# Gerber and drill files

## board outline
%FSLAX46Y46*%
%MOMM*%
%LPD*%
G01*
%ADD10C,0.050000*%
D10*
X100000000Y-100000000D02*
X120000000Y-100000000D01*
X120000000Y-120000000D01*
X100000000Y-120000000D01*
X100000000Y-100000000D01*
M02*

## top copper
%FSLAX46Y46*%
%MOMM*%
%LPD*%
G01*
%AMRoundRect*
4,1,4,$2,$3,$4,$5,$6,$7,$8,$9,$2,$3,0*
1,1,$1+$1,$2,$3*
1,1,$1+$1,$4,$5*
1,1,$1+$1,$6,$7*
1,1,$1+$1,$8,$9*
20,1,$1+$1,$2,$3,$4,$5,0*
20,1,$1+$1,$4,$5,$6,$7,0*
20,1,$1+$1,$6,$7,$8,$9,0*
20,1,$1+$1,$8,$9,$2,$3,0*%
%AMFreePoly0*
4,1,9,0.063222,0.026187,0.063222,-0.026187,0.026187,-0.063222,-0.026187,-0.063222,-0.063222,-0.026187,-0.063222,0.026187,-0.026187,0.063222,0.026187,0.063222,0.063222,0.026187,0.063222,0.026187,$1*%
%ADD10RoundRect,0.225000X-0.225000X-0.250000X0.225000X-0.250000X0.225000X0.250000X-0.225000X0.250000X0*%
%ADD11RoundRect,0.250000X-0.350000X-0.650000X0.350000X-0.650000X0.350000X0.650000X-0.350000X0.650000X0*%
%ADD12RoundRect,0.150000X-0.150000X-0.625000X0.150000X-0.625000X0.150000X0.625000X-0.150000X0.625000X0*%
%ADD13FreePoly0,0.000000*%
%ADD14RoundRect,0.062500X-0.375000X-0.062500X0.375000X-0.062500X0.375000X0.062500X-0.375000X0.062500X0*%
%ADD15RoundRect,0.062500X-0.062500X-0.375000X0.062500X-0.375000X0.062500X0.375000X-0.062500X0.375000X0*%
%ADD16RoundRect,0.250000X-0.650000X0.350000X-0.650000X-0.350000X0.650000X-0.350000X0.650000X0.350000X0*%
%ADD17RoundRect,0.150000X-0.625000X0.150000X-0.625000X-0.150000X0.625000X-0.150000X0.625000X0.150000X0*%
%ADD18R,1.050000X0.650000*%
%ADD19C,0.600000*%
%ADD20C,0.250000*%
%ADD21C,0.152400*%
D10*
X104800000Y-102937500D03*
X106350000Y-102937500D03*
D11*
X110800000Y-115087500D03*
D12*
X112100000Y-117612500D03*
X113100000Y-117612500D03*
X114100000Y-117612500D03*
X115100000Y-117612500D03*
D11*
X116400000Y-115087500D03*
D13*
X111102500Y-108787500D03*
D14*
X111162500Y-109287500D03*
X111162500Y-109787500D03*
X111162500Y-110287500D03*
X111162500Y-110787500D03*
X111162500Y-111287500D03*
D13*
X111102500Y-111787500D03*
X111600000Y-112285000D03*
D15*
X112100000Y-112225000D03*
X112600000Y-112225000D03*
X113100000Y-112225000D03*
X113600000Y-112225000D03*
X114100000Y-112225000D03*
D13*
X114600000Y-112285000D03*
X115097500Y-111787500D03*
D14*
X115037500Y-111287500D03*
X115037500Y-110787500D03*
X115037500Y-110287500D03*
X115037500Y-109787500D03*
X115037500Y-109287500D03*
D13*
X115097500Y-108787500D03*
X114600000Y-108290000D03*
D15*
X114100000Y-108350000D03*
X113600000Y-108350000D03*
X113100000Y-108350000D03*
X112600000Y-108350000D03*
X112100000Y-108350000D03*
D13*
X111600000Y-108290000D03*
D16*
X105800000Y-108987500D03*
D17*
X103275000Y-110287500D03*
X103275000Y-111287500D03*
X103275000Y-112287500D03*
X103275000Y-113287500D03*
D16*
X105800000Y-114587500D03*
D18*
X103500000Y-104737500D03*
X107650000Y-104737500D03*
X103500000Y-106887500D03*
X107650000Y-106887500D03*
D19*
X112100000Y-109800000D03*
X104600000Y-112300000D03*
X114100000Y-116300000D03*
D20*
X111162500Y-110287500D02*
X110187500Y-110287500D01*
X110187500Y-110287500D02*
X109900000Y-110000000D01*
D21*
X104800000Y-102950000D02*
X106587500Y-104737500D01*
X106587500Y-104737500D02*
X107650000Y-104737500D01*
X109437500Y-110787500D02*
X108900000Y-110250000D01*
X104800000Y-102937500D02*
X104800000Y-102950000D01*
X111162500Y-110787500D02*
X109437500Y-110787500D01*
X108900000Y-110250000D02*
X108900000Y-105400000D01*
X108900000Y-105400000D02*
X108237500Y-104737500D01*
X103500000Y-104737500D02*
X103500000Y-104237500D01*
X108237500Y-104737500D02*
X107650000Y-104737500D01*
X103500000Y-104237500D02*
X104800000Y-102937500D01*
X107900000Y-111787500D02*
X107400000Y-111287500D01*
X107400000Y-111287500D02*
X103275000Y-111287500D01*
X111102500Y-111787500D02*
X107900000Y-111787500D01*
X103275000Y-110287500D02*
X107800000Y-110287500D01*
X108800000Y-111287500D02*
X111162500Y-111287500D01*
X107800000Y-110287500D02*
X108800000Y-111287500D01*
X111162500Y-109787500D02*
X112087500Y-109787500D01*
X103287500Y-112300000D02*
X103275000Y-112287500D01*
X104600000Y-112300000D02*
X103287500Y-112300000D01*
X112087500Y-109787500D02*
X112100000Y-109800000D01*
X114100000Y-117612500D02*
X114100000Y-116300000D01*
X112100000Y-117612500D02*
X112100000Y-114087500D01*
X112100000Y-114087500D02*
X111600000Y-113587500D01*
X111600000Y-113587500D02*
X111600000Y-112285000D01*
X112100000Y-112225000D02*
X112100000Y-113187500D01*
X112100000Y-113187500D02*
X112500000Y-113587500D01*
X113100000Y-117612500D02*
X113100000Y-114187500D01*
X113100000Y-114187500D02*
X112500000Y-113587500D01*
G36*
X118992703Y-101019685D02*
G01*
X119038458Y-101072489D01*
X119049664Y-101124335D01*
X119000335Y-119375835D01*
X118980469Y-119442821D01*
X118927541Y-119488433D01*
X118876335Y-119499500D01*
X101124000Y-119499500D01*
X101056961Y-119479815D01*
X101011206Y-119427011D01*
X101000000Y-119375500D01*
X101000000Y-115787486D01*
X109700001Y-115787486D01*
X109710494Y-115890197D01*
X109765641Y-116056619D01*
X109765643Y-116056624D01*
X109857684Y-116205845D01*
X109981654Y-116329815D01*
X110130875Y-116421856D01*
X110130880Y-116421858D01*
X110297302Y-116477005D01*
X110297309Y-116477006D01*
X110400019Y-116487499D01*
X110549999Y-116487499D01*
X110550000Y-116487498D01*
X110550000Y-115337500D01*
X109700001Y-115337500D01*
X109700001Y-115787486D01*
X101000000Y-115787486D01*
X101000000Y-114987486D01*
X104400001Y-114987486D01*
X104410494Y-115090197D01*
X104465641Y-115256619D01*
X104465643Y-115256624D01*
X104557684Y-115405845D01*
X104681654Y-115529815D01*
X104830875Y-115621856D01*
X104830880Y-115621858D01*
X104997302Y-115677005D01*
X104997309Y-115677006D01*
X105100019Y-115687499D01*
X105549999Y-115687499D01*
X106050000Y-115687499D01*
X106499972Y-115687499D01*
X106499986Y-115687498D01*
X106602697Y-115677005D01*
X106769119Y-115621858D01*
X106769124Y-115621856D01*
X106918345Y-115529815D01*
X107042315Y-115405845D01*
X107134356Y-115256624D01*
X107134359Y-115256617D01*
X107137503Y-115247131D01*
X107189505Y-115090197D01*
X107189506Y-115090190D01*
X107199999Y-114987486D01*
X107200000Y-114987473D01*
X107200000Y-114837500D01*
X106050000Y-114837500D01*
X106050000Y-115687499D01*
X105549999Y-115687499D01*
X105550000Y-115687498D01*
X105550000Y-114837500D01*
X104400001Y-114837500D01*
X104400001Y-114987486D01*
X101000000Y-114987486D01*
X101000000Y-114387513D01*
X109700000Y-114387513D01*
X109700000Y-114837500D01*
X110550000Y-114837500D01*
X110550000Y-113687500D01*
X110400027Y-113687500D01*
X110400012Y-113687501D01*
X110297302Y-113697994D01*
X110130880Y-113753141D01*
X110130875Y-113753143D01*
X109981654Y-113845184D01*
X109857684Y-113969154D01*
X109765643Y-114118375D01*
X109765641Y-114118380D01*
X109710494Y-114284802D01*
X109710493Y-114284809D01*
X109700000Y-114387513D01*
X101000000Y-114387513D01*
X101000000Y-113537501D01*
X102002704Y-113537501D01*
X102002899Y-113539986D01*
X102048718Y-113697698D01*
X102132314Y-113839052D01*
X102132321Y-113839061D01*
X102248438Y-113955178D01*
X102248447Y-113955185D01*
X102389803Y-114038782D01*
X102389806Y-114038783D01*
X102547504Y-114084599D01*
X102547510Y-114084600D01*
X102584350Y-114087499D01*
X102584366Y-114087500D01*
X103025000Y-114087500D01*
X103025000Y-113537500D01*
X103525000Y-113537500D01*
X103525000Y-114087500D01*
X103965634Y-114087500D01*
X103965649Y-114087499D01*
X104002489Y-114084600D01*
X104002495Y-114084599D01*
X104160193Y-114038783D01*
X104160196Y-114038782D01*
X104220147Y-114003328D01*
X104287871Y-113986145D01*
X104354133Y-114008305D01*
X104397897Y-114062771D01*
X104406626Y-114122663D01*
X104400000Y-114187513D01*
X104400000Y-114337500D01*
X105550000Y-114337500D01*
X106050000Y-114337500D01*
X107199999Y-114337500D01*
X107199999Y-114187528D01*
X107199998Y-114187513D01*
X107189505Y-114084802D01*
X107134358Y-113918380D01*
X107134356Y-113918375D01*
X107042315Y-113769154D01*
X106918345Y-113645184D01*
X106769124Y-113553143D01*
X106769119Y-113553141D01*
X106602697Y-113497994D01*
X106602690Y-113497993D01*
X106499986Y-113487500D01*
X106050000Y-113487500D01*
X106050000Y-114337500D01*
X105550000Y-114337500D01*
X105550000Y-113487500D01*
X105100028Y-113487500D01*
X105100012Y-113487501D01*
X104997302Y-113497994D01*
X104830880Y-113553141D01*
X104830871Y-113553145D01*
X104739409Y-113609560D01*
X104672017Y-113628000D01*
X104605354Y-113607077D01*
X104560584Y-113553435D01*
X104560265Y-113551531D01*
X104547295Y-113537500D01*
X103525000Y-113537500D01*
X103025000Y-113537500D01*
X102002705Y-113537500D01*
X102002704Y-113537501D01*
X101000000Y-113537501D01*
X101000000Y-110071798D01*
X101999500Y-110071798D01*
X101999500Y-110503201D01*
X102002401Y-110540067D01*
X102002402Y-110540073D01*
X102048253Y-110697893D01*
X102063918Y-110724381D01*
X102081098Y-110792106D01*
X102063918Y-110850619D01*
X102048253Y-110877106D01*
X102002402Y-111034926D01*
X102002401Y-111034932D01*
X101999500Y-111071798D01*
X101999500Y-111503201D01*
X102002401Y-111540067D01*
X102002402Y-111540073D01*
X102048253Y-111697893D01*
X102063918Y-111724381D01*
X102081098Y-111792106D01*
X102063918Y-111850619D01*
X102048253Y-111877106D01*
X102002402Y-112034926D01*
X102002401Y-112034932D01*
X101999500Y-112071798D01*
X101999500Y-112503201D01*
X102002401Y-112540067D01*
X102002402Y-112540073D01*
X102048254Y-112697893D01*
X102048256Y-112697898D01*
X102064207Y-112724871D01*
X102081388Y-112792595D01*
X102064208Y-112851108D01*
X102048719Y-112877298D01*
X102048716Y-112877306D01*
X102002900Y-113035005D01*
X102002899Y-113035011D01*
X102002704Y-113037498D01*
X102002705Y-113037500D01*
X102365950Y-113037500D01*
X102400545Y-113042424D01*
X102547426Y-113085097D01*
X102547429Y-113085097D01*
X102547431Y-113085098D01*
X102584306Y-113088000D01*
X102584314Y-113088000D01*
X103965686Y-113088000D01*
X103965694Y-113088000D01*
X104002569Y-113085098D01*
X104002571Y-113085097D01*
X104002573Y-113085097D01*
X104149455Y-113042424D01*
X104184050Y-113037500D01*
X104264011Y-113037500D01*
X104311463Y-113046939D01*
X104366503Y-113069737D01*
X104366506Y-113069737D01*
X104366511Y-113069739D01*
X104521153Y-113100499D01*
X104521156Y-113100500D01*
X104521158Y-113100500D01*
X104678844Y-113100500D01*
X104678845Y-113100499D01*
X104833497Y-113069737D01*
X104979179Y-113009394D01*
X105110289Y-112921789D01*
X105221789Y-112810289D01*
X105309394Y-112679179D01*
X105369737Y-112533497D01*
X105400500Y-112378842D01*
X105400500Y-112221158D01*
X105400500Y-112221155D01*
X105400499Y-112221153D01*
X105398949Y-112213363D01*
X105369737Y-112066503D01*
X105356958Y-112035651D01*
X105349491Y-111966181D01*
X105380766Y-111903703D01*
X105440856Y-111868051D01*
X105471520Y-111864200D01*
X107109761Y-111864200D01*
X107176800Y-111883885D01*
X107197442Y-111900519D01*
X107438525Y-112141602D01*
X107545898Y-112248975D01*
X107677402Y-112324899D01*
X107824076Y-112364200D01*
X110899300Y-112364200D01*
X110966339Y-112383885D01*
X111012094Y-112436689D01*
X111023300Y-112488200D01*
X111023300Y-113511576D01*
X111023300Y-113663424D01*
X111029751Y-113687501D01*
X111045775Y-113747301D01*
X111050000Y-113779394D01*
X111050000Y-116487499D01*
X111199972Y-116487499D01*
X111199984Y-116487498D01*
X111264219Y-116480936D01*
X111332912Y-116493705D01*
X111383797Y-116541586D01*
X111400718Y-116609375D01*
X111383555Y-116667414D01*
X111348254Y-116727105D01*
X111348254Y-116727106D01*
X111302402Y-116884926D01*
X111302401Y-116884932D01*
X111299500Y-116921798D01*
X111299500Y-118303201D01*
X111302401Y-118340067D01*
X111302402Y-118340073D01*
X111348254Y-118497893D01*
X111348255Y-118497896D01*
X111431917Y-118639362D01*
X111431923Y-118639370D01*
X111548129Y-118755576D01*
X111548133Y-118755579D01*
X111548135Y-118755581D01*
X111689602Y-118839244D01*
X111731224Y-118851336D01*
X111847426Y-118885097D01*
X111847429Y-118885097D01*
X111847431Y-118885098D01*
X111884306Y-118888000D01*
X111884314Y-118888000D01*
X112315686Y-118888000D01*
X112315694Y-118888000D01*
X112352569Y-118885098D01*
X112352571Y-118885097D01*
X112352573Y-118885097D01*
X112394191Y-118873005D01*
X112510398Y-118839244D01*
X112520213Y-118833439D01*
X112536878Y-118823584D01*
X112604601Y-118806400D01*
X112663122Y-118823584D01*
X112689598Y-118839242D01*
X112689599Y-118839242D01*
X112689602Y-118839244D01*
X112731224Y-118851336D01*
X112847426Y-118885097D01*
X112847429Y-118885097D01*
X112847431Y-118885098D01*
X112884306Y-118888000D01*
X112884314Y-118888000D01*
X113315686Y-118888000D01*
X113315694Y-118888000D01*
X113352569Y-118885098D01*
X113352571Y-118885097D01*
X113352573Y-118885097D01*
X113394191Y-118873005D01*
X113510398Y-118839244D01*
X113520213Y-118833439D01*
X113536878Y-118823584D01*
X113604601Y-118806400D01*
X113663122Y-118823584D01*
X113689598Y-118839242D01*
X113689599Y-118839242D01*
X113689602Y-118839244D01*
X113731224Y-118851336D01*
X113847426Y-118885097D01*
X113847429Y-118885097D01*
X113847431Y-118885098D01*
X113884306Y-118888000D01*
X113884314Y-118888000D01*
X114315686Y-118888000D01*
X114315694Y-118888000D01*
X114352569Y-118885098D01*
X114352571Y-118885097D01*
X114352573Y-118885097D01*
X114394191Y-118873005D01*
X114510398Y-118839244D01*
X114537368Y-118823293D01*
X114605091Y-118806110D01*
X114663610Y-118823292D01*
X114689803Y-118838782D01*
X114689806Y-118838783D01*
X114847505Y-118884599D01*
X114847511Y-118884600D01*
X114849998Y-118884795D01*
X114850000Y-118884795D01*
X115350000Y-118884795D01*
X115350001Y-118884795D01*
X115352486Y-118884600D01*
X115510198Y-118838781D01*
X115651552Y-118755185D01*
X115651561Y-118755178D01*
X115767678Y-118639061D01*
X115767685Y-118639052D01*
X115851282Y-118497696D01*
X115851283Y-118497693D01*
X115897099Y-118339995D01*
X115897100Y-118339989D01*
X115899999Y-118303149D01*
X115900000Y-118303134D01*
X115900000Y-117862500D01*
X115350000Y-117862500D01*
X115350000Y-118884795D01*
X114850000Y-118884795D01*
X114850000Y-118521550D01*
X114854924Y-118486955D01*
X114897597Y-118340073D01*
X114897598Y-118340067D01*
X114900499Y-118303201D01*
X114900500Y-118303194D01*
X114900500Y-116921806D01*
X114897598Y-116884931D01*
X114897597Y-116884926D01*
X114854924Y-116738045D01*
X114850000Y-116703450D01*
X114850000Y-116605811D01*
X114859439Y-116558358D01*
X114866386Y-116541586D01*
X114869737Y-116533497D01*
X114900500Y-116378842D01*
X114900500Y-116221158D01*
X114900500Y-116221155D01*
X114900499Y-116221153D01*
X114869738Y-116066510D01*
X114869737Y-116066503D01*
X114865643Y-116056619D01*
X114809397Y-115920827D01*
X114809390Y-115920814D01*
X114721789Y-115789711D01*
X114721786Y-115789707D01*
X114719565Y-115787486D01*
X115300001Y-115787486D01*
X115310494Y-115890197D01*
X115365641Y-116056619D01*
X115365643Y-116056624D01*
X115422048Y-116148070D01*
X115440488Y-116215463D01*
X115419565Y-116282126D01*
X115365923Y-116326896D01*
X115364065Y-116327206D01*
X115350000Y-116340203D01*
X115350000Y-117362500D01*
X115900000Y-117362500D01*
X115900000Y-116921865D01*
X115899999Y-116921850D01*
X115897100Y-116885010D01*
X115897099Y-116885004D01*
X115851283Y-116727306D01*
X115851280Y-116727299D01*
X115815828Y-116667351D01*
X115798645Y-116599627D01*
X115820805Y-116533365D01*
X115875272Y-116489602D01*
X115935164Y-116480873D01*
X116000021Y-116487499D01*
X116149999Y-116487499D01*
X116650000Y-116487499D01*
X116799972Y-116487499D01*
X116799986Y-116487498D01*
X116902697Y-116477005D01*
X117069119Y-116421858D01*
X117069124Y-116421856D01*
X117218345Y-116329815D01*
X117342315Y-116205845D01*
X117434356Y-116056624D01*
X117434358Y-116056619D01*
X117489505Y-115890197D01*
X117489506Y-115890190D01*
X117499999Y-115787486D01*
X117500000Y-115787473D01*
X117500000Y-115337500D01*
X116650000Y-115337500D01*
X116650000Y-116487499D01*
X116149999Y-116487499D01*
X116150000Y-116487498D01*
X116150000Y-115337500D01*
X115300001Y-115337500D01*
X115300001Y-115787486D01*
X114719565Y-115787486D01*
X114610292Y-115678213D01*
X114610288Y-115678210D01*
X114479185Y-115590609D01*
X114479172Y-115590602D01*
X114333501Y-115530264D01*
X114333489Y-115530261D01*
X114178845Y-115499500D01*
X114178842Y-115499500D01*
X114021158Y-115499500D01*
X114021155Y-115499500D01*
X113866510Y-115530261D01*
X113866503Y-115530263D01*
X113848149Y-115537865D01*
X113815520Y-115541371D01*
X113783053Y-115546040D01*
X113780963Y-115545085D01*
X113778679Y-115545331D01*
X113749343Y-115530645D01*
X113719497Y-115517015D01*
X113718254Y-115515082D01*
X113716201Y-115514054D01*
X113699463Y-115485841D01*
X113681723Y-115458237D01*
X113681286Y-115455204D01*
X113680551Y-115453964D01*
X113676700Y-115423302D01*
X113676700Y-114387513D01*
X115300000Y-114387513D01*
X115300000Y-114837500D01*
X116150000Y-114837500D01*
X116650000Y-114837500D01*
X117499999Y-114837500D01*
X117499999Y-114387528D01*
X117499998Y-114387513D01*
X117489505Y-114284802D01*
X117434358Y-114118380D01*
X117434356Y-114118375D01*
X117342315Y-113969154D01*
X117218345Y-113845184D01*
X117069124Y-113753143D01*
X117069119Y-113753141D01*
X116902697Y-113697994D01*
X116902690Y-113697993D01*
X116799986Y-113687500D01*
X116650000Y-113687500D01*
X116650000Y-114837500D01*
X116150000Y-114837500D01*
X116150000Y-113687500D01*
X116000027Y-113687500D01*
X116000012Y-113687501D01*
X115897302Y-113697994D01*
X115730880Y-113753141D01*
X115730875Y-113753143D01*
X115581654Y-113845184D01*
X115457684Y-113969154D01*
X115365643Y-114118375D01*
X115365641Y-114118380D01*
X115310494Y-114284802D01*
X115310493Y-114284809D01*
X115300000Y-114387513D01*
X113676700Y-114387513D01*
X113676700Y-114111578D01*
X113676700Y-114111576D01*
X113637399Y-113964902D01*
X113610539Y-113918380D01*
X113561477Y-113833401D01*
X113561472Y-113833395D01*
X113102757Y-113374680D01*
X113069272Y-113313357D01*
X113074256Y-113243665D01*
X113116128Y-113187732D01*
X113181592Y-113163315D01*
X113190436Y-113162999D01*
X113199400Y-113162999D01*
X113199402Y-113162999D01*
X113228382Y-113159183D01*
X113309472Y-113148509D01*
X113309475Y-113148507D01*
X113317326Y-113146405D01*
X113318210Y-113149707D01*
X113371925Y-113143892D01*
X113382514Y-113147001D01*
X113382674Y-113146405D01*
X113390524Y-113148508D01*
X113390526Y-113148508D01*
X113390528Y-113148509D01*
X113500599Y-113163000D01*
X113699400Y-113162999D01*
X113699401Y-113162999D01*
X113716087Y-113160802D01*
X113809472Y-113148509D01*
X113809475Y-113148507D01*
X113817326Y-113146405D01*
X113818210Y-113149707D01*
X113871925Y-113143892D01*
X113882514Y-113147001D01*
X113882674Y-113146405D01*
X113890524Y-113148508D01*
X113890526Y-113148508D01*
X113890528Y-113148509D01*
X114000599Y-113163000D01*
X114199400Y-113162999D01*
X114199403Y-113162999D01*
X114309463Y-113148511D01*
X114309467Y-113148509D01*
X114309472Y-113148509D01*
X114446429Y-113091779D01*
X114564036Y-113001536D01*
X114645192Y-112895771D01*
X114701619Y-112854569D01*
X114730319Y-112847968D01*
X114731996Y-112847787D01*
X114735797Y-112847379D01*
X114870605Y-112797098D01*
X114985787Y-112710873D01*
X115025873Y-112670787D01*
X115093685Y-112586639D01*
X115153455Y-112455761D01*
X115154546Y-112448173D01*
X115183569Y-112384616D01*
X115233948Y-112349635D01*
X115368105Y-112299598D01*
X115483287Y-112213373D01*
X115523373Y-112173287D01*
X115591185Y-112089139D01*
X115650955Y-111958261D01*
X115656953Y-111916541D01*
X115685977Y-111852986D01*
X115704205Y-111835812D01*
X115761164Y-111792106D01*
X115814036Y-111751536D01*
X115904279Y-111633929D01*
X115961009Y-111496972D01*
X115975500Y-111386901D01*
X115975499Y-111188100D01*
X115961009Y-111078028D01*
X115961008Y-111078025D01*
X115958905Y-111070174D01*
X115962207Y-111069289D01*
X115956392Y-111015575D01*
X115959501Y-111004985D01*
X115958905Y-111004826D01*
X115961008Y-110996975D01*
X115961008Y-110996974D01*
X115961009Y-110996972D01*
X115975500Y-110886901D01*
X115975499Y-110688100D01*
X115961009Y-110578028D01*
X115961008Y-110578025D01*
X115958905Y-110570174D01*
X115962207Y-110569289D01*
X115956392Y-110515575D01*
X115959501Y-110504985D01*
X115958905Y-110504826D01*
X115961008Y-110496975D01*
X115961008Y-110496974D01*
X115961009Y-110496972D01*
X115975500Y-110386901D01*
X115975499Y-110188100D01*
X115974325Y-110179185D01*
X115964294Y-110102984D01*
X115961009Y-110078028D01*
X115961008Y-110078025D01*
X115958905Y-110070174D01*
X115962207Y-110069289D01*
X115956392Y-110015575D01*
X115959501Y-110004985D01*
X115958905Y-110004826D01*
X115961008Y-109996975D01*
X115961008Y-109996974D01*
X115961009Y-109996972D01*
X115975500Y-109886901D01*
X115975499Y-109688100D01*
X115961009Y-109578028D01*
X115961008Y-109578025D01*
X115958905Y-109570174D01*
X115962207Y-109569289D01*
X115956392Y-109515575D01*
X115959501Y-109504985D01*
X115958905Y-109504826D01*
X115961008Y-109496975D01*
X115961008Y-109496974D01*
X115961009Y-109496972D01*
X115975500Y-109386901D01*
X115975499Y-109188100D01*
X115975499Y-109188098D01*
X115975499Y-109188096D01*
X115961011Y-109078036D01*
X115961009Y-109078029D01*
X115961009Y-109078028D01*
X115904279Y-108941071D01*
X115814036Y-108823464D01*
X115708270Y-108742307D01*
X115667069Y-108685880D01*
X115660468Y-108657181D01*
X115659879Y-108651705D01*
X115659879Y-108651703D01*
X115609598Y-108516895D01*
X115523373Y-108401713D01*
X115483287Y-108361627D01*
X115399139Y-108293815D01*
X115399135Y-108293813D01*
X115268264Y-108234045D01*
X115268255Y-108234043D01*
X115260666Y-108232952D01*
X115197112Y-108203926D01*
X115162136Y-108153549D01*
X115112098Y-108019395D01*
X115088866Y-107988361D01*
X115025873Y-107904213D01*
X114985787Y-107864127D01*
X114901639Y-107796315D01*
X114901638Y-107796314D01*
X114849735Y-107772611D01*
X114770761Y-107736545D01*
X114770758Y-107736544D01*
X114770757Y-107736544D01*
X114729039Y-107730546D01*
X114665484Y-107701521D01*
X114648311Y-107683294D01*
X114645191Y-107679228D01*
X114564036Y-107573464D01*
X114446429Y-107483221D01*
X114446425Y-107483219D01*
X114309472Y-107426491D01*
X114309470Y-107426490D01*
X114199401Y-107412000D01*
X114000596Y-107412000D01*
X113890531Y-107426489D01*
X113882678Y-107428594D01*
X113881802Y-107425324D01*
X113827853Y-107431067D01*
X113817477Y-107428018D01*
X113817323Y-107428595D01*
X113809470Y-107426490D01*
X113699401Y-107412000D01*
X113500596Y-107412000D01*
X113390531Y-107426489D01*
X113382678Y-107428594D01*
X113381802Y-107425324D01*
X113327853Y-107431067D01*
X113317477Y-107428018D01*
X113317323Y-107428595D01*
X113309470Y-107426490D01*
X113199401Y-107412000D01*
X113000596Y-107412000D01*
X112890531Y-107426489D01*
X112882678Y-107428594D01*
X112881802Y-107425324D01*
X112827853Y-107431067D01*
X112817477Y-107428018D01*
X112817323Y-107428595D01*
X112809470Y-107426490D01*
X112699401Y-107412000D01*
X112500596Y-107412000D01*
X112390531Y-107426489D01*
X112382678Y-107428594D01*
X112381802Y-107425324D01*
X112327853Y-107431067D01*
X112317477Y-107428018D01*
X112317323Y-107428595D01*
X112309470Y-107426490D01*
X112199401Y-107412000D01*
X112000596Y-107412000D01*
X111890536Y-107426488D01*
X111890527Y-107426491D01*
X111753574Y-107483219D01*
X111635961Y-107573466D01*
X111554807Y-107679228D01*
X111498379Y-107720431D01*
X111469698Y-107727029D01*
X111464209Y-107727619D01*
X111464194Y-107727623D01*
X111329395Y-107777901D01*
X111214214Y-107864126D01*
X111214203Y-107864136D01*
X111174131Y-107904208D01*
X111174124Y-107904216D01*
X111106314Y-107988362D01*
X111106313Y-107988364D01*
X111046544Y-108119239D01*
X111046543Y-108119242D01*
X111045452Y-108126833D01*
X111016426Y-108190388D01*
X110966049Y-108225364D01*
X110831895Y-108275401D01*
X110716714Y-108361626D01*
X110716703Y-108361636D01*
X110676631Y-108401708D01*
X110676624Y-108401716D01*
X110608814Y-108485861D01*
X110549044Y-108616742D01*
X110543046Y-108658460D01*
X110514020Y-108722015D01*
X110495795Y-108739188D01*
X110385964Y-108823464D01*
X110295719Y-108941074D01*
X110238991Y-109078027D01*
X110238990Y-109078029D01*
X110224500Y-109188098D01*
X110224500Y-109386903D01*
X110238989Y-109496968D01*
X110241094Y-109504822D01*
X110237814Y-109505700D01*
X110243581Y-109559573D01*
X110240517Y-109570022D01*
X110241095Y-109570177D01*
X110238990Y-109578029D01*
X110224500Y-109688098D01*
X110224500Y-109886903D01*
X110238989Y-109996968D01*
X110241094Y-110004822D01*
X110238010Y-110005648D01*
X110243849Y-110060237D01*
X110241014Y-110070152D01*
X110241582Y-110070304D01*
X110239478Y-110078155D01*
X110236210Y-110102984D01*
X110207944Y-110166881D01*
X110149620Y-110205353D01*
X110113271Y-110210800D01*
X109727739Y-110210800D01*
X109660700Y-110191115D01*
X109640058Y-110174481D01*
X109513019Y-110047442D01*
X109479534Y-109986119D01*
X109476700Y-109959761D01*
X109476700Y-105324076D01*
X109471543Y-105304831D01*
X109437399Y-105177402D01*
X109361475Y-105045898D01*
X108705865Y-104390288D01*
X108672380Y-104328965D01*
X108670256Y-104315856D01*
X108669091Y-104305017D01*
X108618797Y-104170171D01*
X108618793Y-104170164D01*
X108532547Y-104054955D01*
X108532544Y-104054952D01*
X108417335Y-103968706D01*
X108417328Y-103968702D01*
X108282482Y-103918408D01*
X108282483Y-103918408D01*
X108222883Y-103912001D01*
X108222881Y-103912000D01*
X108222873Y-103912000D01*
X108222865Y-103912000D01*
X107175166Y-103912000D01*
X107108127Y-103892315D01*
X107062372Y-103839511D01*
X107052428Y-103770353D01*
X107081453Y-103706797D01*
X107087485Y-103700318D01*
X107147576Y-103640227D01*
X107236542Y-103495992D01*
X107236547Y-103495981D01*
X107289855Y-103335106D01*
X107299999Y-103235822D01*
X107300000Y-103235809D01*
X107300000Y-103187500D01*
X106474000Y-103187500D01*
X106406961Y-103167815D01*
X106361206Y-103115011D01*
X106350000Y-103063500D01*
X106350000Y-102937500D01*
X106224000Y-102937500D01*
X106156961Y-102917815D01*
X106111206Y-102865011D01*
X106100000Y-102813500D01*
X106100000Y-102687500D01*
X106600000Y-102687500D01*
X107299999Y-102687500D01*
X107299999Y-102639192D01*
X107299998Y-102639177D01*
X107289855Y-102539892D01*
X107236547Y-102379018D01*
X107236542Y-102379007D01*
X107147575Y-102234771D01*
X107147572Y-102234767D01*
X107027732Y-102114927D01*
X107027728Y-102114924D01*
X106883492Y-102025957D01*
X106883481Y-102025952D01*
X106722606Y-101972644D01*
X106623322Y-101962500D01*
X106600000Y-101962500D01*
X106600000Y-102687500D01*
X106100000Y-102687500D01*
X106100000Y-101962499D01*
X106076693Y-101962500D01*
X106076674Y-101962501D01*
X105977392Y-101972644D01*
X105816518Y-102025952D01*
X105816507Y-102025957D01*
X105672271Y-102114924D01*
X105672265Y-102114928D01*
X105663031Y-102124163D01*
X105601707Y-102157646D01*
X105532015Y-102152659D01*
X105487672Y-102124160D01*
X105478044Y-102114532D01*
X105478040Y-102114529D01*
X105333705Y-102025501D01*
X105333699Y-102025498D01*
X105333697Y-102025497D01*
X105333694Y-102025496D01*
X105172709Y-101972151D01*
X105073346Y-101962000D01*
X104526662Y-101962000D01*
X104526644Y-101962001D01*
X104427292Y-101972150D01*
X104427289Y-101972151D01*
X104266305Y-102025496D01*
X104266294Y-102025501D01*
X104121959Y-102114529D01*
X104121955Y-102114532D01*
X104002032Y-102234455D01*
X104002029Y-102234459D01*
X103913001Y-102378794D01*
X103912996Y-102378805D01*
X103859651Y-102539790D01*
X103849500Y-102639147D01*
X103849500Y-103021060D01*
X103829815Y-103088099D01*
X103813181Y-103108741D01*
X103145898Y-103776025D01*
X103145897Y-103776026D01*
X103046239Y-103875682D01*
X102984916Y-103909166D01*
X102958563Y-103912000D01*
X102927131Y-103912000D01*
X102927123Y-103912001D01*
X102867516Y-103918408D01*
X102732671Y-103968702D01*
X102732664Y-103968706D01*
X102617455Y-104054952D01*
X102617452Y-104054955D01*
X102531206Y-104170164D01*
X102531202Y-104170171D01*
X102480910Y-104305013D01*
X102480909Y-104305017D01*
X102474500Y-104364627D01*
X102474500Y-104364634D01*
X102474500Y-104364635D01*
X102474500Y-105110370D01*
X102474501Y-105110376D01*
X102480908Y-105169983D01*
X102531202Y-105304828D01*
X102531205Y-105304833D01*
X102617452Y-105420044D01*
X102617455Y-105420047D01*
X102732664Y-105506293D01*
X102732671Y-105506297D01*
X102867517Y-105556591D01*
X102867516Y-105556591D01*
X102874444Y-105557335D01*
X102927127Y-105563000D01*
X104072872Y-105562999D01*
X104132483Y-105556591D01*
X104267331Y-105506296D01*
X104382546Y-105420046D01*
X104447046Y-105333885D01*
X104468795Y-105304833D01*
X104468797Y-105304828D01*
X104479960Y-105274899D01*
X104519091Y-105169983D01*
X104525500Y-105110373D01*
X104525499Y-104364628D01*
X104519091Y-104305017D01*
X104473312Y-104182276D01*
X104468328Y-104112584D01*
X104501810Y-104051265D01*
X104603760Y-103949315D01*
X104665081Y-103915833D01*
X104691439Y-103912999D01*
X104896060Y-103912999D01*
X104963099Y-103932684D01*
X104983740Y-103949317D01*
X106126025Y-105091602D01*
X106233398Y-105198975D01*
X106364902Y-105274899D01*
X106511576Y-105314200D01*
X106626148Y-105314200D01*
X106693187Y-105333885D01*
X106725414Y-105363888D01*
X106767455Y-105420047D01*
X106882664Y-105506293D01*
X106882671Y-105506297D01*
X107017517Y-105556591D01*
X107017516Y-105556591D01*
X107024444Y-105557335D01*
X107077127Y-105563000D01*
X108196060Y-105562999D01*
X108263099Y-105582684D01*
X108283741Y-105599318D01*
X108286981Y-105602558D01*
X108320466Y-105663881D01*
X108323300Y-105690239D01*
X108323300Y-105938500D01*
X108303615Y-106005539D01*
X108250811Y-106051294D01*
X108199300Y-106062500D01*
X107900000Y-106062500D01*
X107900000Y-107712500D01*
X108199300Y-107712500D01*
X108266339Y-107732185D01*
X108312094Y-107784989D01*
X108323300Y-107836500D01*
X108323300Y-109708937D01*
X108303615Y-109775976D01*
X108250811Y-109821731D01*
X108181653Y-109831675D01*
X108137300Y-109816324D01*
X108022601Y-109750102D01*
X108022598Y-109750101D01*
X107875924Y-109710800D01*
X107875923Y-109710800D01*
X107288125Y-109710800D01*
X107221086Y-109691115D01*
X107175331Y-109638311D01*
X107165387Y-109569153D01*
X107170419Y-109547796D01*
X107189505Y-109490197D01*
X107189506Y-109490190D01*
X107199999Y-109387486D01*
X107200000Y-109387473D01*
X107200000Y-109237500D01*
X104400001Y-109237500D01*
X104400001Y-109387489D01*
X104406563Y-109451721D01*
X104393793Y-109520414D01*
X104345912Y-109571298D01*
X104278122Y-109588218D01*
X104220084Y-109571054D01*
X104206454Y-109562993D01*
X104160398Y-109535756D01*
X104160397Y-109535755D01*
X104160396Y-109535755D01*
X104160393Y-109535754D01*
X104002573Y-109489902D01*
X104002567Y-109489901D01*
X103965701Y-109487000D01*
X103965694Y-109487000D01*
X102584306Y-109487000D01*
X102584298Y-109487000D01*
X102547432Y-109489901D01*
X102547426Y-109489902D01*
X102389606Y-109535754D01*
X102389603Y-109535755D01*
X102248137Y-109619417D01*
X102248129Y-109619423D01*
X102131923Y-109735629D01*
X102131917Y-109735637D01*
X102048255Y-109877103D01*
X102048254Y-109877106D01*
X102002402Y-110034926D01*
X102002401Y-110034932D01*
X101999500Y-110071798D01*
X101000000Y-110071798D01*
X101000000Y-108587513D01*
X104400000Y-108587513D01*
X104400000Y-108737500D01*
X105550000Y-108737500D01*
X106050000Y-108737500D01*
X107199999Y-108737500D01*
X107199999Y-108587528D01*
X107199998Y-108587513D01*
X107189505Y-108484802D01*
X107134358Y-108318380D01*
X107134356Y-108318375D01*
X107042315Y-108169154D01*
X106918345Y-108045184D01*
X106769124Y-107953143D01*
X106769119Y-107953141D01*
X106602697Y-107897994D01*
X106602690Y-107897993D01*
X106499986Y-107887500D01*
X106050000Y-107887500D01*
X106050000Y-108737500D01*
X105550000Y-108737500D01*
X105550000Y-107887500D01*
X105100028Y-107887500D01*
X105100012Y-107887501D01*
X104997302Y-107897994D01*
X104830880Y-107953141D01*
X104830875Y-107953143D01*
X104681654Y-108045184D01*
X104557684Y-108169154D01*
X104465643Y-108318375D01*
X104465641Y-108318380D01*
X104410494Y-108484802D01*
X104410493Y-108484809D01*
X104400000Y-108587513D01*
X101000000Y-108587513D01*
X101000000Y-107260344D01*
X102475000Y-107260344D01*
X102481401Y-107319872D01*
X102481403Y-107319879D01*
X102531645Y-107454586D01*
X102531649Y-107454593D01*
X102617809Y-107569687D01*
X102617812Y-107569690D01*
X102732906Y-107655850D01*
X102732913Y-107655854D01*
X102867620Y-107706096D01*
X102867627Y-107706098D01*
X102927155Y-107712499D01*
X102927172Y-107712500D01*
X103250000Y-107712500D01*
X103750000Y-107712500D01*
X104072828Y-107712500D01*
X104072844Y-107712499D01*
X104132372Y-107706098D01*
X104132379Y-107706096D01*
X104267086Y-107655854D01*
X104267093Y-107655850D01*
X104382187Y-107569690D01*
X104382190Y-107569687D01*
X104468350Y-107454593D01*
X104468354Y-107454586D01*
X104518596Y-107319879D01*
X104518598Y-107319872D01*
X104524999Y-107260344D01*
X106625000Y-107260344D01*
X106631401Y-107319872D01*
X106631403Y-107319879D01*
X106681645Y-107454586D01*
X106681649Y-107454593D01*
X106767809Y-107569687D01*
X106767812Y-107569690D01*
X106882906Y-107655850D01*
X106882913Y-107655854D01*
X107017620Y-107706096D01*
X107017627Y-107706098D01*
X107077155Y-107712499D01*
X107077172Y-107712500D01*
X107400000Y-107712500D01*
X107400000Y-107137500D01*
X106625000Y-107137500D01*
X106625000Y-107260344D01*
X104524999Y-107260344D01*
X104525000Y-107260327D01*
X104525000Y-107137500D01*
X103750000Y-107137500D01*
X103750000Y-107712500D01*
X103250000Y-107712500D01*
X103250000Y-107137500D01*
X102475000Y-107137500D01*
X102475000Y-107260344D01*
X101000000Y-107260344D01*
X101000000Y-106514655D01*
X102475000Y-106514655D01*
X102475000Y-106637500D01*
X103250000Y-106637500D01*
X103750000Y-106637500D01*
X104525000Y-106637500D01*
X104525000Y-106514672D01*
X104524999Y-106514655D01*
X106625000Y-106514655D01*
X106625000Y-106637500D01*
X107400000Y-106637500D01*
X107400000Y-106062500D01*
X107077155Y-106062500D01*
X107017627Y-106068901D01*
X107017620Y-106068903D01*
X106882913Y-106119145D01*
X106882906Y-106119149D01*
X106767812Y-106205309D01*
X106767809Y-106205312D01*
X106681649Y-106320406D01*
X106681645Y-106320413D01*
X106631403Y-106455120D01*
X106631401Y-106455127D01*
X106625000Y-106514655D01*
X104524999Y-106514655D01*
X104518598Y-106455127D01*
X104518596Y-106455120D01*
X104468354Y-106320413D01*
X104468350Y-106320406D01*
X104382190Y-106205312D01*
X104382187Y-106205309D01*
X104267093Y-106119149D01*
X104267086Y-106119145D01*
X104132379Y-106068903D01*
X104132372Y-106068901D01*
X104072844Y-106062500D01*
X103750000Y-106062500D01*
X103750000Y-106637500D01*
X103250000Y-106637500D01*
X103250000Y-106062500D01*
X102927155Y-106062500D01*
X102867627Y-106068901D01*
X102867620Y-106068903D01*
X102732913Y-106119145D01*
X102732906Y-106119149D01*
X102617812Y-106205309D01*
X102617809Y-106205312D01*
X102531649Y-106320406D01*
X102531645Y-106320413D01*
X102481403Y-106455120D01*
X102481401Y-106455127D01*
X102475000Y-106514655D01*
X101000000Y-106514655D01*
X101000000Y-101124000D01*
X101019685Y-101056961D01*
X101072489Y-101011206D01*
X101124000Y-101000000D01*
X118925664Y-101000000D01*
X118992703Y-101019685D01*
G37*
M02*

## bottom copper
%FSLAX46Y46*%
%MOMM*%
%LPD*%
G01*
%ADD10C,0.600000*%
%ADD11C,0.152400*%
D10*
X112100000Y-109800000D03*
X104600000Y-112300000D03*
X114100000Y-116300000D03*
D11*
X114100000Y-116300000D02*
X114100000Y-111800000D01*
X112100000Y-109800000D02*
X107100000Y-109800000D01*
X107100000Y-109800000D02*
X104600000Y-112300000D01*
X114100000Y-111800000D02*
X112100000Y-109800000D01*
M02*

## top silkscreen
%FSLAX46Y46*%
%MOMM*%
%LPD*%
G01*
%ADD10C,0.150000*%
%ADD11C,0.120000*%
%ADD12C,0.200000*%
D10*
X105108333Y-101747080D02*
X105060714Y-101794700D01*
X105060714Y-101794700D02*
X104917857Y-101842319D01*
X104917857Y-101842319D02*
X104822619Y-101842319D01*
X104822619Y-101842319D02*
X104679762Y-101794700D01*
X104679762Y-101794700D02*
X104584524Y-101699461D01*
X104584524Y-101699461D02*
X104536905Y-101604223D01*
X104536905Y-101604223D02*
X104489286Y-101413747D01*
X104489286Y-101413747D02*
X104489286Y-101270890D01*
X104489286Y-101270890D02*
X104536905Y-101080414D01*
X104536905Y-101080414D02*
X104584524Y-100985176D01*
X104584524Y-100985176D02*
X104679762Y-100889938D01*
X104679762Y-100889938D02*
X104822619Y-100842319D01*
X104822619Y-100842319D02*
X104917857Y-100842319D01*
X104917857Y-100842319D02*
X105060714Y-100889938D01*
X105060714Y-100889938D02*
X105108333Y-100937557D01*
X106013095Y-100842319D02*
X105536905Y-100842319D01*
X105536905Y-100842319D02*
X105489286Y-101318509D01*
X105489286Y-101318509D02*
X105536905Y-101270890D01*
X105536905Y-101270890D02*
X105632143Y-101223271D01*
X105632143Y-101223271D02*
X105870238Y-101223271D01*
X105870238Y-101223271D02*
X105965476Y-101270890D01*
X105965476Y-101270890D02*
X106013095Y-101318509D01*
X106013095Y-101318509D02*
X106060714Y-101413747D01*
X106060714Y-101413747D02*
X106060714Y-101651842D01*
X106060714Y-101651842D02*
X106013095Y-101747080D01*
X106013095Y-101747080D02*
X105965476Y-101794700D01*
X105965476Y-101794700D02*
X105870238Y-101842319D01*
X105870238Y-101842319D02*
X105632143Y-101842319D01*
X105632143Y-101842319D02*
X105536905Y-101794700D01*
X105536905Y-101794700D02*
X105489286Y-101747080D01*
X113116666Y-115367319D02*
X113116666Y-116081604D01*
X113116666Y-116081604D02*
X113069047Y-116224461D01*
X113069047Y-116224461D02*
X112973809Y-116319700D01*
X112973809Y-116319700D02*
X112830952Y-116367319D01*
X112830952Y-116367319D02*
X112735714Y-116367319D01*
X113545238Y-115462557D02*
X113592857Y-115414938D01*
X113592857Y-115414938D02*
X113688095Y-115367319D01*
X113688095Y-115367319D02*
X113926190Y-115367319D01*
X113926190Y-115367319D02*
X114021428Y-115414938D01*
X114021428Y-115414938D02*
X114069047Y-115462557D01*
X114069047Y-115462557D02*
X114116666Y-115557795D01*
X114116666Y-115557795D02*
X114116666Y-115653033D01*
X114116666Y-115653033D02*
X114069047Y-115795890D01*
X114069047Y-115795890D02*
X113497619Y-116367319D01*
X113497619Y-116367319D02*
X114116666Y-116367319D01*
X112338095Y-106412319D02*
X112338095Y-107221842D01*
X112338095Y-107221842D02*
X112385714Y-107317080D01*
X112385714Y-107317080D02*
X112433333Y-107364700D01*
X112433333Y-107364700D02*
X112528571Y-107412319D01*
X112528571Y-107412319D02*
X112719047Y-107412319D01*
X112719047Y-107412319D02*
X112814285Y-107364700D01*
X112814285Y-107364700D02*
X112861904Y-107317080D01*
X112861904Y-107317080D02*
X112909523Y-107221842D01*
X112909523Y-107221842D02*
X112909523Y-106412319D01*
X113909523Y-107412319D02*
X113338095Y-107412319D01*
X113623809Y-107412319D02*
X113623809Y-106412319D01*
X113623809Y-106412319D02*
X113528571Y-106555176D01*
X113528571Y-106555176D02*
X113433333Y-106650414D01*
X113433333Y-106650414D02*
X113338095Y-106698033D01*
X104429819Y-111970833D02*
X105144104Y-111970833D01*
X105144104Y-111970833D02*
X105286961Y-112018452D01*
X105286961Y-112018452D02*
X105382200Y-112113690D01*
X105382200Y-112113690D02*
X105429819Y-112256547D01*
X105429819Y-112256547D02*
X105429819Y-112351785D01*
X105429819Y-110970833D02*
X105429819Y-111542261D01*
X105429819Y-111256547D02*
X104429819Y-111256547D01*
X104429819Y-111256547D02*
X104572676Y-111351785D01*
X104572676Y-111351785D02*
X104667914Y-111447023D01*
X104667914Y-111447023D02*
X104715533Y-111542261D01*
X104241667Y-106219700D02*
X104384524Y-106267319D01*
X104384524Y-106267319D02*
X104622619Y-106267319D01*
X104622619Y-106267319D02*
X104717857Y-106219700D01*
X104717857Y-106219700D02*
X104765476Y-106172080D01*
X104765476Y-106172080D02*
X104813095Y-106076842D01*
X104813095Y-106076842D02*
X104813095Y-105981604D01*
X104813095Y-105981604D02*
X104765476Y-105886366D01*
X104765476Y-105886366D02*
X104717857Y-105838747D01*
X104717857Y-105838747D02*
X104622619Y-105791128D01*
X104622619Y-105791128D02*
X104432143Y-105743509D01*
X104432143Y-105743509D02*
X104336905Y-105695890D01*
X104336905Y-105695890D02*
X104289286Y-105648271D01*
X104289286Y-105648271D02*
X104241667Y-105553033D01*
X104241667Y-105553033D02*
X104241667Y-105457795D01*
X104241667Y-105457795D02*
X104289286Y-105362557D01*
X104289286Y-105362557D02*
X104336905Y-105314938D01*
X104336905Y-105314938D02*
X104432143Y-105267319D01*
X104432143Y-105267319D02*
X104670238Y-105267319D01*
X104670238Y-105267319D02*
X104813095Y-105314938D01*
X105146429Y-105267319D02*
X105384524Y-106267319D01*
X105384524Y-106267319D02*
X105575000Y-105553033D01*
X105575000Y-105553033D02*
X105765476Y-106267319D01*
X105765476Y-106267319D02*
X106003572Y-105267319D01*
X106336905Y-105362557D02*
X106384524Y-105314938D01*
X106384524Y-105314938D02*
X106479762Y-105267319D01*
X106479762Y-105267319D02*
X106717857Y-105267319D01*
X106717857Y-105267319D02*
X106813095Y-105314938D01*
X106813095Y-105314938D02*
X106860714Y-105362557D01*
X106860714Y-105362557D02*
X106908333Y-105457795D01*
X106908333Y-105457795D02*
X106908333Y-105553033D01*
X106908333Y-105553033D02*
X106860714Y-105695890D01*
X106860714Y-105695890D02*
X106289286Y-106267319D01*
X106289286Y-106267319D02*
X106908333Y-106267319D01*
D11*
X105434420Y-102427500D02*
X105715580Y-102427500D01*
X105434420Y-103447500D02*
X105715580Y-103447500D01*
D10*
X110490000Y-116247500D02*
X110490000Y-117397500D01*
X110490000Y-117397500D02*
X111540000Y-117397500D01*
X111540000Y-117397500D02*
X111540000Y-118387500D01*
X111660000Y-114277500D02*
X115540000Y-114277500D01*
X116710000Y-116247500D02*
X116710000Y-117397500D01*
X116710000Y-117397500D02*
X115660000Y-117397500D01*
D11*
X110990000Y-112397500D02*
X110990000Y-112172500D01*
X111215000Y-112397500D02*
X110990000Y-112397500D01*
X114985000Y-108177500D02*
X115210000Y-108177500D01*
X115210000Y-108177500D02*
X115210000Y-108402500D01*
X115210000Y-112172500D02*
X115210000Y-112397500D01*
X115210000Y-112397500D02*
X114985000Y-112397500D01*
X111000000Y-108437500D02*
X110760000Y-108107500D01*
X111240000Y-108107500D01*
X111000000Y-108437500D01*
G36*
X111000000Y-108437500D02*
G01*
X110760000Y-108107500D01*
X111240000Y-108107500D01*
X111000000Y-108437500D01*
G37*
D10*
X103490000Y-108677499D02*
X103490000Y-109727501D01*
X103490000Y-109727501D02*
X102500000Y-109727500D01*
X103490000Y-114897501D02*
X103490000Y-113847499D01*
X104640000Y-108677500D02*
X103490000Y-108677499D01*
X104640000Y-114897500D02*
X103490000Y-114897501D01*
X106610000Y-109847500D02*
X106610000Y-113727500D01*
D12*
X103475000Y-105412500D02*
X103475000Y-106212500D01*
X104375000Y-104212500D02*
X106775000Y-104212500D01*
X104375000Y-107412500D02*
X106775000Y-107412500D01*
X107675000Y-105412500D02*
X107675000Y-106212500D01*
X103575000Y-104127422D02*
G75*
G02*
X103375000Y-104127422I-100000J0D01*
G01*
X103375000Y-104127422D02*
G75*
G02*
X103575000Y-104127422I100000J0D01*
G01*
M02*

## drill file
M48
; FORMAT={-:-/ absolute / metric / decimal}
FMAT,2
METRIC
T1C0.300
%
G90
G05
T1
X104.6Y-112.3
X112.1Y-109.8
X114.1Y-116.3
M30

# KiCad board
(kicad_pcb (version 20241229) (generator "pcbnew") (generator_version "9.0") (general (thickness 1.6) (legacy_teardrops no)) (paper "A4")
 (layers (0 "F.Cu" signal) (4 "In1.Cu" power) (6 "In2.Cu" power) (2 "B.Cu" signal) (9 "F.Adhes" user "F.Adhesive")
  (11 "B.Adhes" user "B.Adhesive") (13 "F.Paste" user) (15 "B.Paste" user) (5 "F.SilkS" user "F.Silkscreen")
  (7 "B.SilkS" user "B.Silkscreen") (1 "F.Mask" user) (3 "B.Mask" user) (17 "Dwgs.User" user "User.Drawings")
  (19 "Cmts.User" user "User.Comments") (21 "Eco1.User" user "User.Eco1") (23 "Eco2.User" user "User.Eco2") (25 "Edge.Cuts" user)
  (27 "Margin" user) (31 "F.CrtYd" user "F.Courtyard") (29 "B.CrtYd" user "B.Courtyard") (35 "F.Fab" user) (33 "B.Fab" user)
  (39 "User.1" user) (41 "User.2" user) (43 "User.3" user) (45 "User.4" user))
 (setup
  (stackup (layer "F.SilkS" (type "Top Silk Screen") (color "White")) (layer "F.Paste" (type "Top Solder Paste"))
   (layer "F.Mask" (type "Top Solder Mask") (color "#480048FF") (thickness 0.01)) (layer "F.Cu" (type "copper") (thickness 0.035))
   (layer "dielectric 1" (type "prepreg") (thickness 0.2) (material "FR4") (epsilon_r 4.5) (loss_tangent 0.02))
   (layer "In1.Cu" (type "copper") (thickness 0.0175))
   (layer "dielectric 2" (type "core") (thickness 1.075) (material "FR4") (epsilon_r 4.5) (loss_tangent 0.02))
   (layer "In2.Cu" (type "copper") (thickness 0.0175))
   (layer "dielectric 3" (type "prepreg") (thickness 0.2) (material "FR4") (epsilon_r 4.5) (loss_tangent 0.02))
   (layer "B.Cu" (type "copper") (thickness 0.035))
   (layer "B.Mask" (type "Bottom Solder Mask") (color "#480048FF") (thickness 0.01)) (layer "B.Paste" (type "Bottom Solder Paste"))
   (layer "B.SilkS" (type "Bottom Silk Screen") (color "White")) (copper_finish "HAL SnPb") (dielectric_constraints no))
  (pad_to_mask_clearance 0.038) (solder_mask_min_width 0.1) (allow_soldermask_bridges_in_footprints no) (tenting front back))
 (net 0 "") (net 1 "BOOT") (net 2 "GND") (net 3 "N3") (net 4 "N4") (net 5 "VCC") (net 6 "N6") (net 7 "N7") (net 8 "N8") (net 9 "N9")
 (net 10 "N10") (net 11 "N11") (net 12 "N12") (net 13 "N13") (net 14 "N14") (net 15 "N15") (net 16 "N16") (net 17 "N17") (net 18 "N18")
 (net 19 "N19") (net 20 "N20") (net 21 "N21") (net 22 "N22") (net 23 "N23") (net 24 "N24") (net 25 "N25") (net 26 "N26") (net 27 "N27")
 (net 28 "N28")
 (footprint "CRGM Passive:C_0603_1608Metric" (layer "F.Cu") (at 105.575 102.9375)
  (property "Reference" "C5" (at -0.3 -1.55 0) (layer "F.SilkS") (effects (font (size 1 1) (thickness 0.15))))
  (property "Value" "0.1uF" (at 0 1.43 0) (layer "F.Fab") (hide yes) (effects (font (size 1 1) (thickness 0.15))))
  (fp_line (start -0.14058 -0.51) (end 0.14058 -0.51) (stroke (width 0.12) (type solid)) (layer "F.SilkS"))
  (fp_line (start -0.14058 0.51) (end 0.14058 0.51) (stroke (width 0.12) (type solid)) (layer "F.SilkS"))
  (pad "1" smd roundrect (at -0.775 0) (size 0.9 0.95) (layers "F.Cu" "F.Mask" "F.Paste") (roundrect_rratio 0.25) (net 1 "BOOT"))
  (pad "2" smd roundrect (at 0.775 0) (size 0.9 0.95) (layers "F.Cu" "F.Mask" "F.Paste") (roundrect_rratio 0.25) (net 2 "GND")))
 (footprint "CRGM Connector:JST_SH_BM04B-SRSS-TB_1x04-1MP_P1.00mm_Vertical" (layer "F.Cu") (at 113.6 116.2875)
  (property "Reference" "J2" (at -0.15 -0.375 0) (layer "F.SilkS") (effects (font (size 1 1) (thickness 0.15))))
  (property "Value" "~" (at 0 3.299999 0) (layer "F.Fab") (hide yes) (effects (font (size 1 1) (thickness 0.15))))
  (fp_line (start -3.11 -0.04) (end -3.11 1.11) (stroke (width 0.15) (type solid)) (layer "F.SilkS"))
  (fp_line (start -3.11 1.11) (end -2.06 1.11) (stroke (width 0.15) (type solid)) (layer "F.SilkS"))
  (fp_line (start -2.06 1.11) (end -2.06 2.1) (stroke (width 0.15) (type solid)) (layer "F.SilkS"))
  (fp_line (start -1.94 -2.01) (end 1.94 -2.01) (stroke (width 0.15) (type solid)) (layer "F.SilkS"))
  (fp_line (start 3.11 -0.04) (end 3.11 1.11) (stroke (width 0.15) (type solid)) (layer "F.SilkS"))
  (fp_line (start 3.11 1.11) (end 2.06 1.11) (stroke (width 0.15) (type solid)) (layer "F.SilkS"))
  (pad "0" smd roundrect (at -2.8 -1.2) (size 1.2 1.8) (layers "F.Cu" "F.Mask" "F.Paste") (roundrect_rratio 0.208333) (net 2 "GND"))
  (pad "1" smd roundrect (at -1.5 1.325) (size 0.6 1.55) (layers "F.Cu" "F.Mask" "F.Paste") (roundrect_rratio 0.25) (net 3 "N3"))
  (pad "2" smd roundrect (at -0.5 1.325) (size 0.6 1.55) (layers "F.Cu" "F.Mask" "F.Paste") (roundrect_rratio 0.25) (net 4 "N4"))
  (pad "3" smd roundrect (at 0.5 1.325) (size 0.6 1.55) (layers "F.Cu" "F.Mask" "F.Paste") (roundrect_rratio 0.25) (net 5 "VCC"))
  (pad "4" smd roundrect (at 1.5 1.325) (size 0.6 1.55) (layers "F.Cu" "F.Mask" "F.Paste") (roundrect_rratio 0.25) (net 2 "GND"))
  (pad "5" smd roundrect (at 2.8 -1.2) (size 1.2 1.8) (layers "F.Cu" "F.Mask" "F.Paste") (roundrect_rratio 0.208333) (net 2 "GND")))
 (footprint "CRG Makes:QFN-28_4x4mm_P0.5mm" (layer "F.Cu") (at 113.1 110.2875)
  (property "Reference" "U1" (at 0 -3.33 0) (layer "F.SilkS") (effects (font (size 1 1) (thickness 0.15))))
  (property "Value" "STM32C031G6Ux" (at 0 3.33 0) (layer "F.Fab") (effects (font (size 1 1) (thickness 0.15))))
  (fp_line (start -2.11 2.11) (end -2.11 1.885) (stroke (width 0.12) (type solid)) (layer "F.SilkS"))
  (fp_line (start -1.885 2.11) (end -2.11 2.11) (stroke (width 0.12) (type solid)) (layer "F.SilkS"))
  (fp_line (start 1.885 -2.11) (end 2.11 -2.11) (stroke (width 0.12) (type solid)) (layer "F.SilkS"))
  (fp_line (start 2.11 -2.11) (end 2.11 -1.885) (stroke (width 0.12) (type solid)) (layer "F.SilkS"))
  (fp_line (start 2.11 1.885) (end 2.11 2.11) (stroke (width 0.12) (type solid)) (layer "F.SilkS"))
  (fp_line (start 2.11 2.11) (end 1.885 2.11) (stroke (width 0.12) (type solid)) (layer "F.SilkS"))
  (fp_poly (pts (xy -2.1 -1.85) (xy -2.34 -2.18) (xy -1.86 -2.18)) (stroke (width 0.12) (type solid)) (fill yes) (layer "F.SilkS"))
  (pad "1" smd custom (at -1.9975 -1.5) (size 0.136863 0.136863) (layers "F.Cu" "F.Mask" "F.Paste") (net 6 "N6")
   (options (clearance outline) (anchor circle)) (primitives))
  (pad "2" smd roundrect (at -1.9375 -1) (size 0.875 0.25) (layers "F.Cu" "F.Mask" "F.Paste") (roundrect_rratio 0.25) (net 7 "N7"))
  (pad "3" smd roundrect (at -1.9375 -0.5) (size 0.875 0.25) (layers "F.Cu" "F.Mask" "F.Paste") (roundrect_rratio 0.25) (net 5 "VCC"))
  (pad "4" smd roundrect (at -1.9375 0) (size 0.875 0.25) (layers "F.Cu" "F.Mask" "F.Paste") (roundrect_rratio 0.25) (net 2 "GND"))
  (pad "5" smd roundrect (at -1.9375 0.5) (size 0.875 0.25) (layers "F.Cu" "F.Mask" "F.Paste") (roundrect_rratio 0.25) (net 1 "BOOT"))
  (pad "6" smd roundrect (at -1.9375 1) (size 0.875 0.25) (layers "F.Cu" "F.Mask" "F.Paste") (roundrect_rratio 0.25) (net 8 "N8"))
  (pad "7" smd custom (at -1.9975 1.5) (size 0.136863 0.136863) (layers "F.Cu" "F.Mask" "F.Paste") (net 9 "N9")
   (options (clearance outline) (anchor circle)) (primitives))
  (pad "8" smd custom (at -1.5 1.9975) (size 0.136863 0.136863) (layers "F.Cu" "F.Mask" "F.Paste") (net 3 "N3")
   (options (clearance outline) (anchor circle)) (primitives))
  (pad "9" smd roundrect (at -1 1.9375) (size 0.25 0.875) (layers "F.Cu" "F.Mask" "F.Paste") (roundrect_rratio 0.25) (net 4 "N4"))
  (pad "10" smd roundrect (at -0.5 1.9375) (size 0.25 0.875) (layers "F.Cu" "F.Mask" "F.Paste") (roundrect_rratio 0.25) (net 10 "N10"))
  (pad "11" smd roundrect (at 0 1.9375) (size 0.25 0.875) (layers "F.Cu" "F.Mask" "F.Paste") (roundrect_rratio 0.25) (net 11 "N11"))
  (pad "12" smd roundrect (at 0.5 1.9375) (size 0.25 0.875) (layers "F.Cu" "F.Mask" "F.Paste") (roundrect_rratio 0.25) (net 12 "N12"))
  (pad "13" smd roundrect (at 1 1.9375) (size 0.25 0.875) (layers "F.Cu" "F.Mask" "F.Paste") (roundrect_rratio 0.25) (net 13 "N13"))
  (pad "14" smd custom (at 1.5 1.9975) (size 0.136863 0.136863) (layers "F.Cu" "F.Mask" "F.Paste") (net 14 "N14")
   (options (clearance outline) (anchor circle)) (primitives))
  (pad "15" smd custom (at 1.9975 1.5) (size 0.136863 0.136863) (layers "F.Cu" "F.Mask" "F.Paste") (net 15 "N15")
   (options (clearance outline) (anchor circle)) (primitives))
  (pad "16" smd roundrect (at 1.9375 1) (size 0.875 0.25) (layers "F.Cu" "F.Mask" "F.Paste") (roundrect_rratio 0.25) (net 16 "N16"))
  (pad "17" smd roundrect (at 1.9375 0.5) (size 0.875 0.25) (layers "F.Cu" "F.Mask" "F.Paste") (roundrect_rratio 0.25) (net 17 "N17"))
  (pad "18" smd roundrect (at 1.9375 0) (size 0.875 0.25) (layers "F.Cu" "F.Mask" "F.Paste") (roundrect_rratio 0.25) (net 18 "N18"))
  (pad "19" smd roundrect (at 1.9375 -0.5) (size 0.875 0.25) (layers "F.Cu" "F.Mask" "F.Paste") (roundrect_rratio 0.25) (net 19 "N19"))
  (pad "20" smd roundrect (at 1.9375 -1) (size 0.875 0.25) (layers "F.Cu" "F.Mask" "F.Paste") (roundrect_rratio 0.25) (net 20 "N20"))
  (pad "21" smd custom (at 1.9975 -1.5) (size 0.136863 0.136863) (layers "F.Cu" "F.Mask" "F.Paste") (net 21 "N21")
   (options (clearance outline) (anchor circle)) (primitives))
  (pad "22" smd custom (at 1.5 -1.9975) (size 0.136863 0.136863) (layers "F.Cu" "F.Mask" "F.Paste") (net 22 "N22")
   (options (clearance outline) (anchor circle)) (primitives))
  (pad "23" smd roundrect (at 1 -1.9375) (size 0.25 0.875) (layers "F.Cu" "F.Mask" "F.Paste") (roundrect_rratio 0.25) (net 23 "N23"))
  (pad "24" smd roundrect (at 0.5 -1.9375) (size 0.25 0.875) (layers "F.Cu" "F.Mask" "F.Paste") (roundrect_rratio 0.25) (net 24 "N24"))
  (pad "25" smd roundrect (at 0 -1.9375) (size 0.25 0.875) (layers "F.Cu" "F.Mask" "F.Paste") (roundrect_rratio 0.25) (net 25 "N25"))
  (pad "26" smd roundrect (at -0.5 -1.9375) (size 0.25 0.875) (layers "F.Cu" "F.Mask" "F.Paste") (roundrect_rratio 0.25) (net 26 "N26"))
  (pad "27" smd roundrect (at -1 -1.9375) (size 0.25 0.875) (layers "F.Cu" "F.Mask" "F.Paste") (roundrect_rratio 0.25) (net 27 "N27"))
  (pad "28" smd custom (at -1.5 -1.9975) (size 0.136863 0.136863) (layers "F.Cu" "F.Mask" "F.Paste") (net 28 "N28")
   (options (clearance outline) (anchor circle)) (primitives)))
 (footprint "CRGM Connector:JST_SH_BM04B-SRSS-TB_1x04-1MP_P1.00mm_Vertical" (layer "F.Cu") (at 104.6 111.7875 -90)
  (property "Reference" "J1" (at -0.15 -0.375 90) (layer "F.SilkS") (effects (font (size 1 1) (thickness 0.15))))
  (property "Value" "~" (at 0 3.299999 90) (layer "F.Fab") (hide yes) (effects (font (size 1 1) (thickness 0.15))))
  (fp_line (start -3.110001 1.11) (end -2.059999 1.11) (stroke (width 0.15) (type solid)) (layer "F.SilkS"))
  (fp_line (start -2.059999 1.11) (end -2.06 2.1) (stroke (width 0.15) (type solid)) (layer "F.SilkS"))
  (fp_line (start 3.110001 1.11) (end 2.059999 1.11) (stroke (width 0.15) (type solid)) (layer "F.SilkS"))
  (fp_line (start -3.11 -0.04) (end -3.110001 1.11) (stroke (width 0.15) (type solid)) (layer "F.SilkS"))
  (fp_line (start 3.11 -0.04) (end 3.110001 1.11) (stroke (width 0.15) (type solid)) (layer "F.SilkS"))
  (fp_line (start -1.94 -2.01) (end 1.94 -2.01) (stroke (width 0.15) (type solid)) (layer "F.SilkS"))
  (pad "0" smd roundrect (at -2.8 -1.2 270) (size 1.2 1.8) (layers "F.Cu" "F.Mask" "F.Paste") (roundrect_rratio 0.208333) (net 2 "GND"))
  (pad "1" smd roundrect (at -1.5 1.325 270) (size 0.6 1.55) (layers "F.Cu" "F.Mask" "F.Paste") (roundrect_rratio 0.25) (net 8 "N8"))
  (pad "2" smd roundrect (at -0.5 1.325 270) (size 0.6 1.55) (layers "F.Cu" "F.Mask" "F.Paste") (roundrect_rratio 0.25) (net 9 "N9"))
  (pad "3" smd roundrect (at 0.5 1.325 270) (size 0.6 1.55) (layers "F.Cu" "F.Mask" "F.Paste") (roundrect_rratio 0.25) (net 5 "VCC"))
  (pad "4" smd roundrect (at 1.5 1.325 270) (size 0.6 1.55) (layers "F.Cu" "F.Mask" "F.Paste") (roundrect_rratio 0.25) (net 2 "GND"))
  (pad "5" smd roundrect (at 2.8 -1.2 270) (size 1.2 1.8) (layers "F.Cu" "F.Mask" "F.Paste") (roundrect_rratio 0.208333) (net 2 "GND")))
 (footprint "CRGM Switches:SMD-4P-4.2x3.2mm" (layer "F.Cu") (at 105.575 105.8125)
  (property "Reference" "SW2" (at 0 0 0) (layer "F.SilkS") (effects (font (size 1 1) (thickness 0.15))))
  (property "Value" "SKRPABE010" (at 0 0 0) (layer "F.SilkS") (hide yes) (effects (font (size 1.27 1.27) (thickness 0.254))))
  (fp_line (start -2.1 -0.4) (end -2.1 0.4) (stroke (width 0.2) (type solid)) (layer "F.SilkS"))
  (fp_line (start -1.2 -1.6) (end 1.2 -1.6) (stroke (width 0.2) (type solid)) (layer "F.SilkS"))
  (fp_line (start -1.2 1.6) (end 1.2 1.6) (stroke (width 0.2) (type solid)) (layer "F.SilkS"))
  (fp_line (start 2.1 -0.4) (end 2.1 0.4) (stroke (width 0.2) (type solid)) (layer "F.SilkS"))
  (fp_circle (center -2.1 -1.685078) (end -1.95 -1.685078) (stroke (width 0.1) (type default)) (fill yes) (layer "F.SilkS"))
  (pad "1" smd rect (at -2.075 -1.075 90) (size 0.65 1.05) (layers "F.Cu" "F.Mask" "F.Paste") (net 1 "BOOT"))
  (pad "2" smd rect (at 2.075 -1.075 90) (size 0.65 1.05) (layers "F.Cu" "F.Mask" "F.Paste") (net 1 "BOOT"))
  (pad "3" smd rect (at -2.075 1.075 90) (size 0.65 1.05) (layers "F.Cu" "F.Mask" "F.Paste") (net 2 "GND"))
  (pad "4" smd rect (at 2.075 1.075 90) (size 0.65 1.05) (layers "F.Cu" "F.Mask" "F.Paste") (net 2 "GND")))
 (gr_rect (start 100 100) (end 120 120) (stroke (width 0.05) (type default)) (fill no) (layer "Edge.Cuts"))
 (segment (start 111.1625 110.2875) (end 110.1875 110.2875) (width 0.25) (layer "F.Cu") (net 2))
 (segment (start 110.1875 110.2875) (end 109.9 110) (width 0.25) (layer "F.Cu") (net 2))
 (segment (start 104.8 102.95) (end 106.5875 104.7375) (width 0.1524) (layer "F.Cu") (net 1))
 (segment (start 106.5875 104.7375) (end 107.65 104.7375) (width 0.1524) (layer "F.Cu") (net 1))
 (segment (start 109.4375 110.7875) (end 108.9 110.25) (width 0.1524) (layer "F.Cu") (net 1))
 (segment (start 104.8 102.9375) (end 104.8 102.95) (width 0.1524) (layer "F.Cu") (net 1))
 (segment (start 111.1625 110.7875) (end 109.4375 110.7875) (width 0.1524) (layer "F.Cu") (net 1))
 (segment (start 108.9 110.25) (end 108.9 105.4) (width 0.1524) (layer "F.Cu") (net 1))
 (segment (start 108.9 105.4) (end 108.2375 104.7375) (width 0.1524) (layer "F.Cu") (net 1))
 (segment (start 103.5 104.7375) (end 103.5 104.2375) (width 0.1524) (layer "F.Cu") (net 1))
 (segment (start 108.2375 104.7375) (end 107.65 104.7375) (width 0.1524) (layer "F.Cu") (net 1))
 (segment (start 103.5 104.2375) (end 104.8 102.9375) (width 0.1524) (layer "F.Cu") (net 1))
 (segment (start 107.9 111.7875) (end 107.4 111.2875) (width 0.1524) (layer "F.Cu") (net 9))
 (segment (start 107.4 111.2875) (end 103.275 111.2875) (width 0.1524) (layer "F.Cu") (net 9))
 (segment (start 111.1025 111.7875) (end 107.9 111.7875) (width 0.1524) (layer "F.Cu") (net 9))
 (segment (start 103.275 110.2875) (end 107.8 110.2875) (width 0.1524) (layer "F.Cu") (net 8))
 (segment (start 108.8 111.2875) (end 111.1625 111.2875) (width 0.1524) (layer "F.Cu") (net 8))
 (segment (start 107.8 110.2875) (end 108.8 111.2875) (width 0.1524) (layer "F.Cu") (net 8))
 (segment (start 111.1625 109.7875) (end 112.0875 109.7875) (width 0.1524) (layer "F.Cu") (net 5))
 (segment (start 103.2875 112.3) (end 103.275 112.2875) (width 0.1524) (layer "F.Cu") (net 5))
 (segment (start 104.6 112.3) (end 103.2875 112.3) (width 0.1524) (layer "F.Cu") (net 5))
 (segment (start 112.0875 109.7875) (end 112.1 109.8) (width 0.1524) (layer "F.Cu") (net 5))
 (segment (start 114.1 117.6125) (end 114.1 116.3) (width 0.1524) (layer "F.Cu") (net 5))
 (via (at 112.1 109.8) (size 0.6) (drill 0.3) (layers "F.Cu" "B.Cu") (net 5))
 (via (at 104.6 112.3) (size 0.6) (drill 0.3) (layers "F.Cu" "B.Cu") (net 5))
 (via (at 114.1 116.3) (size 0.6) (drill 0.3) (layers "F.Cu" "B.Cu") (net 5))
 (segment (start 114.1 116.3) (end 114.1 111.8) (width 0.1524) (layer "B.Cu") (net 5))
 (segment (start 112.1 109.8) (end 107.1 109.8) (width 0.1524) (layer "B.Cu") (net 5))
 (segment (start 107.1 109.8) (end 104.6 112.3) (width 0.1524) (layer "B.Cu") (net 5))
 (segment (start 114.1 111.8) (end 112.1 109.8) (width 0.1524) (layer "B.Cu") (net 5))
 (segment (start 112.1 117.6125) (end 112.1 114.0875) (width 0.1524) (layer "F.Cu") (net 3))
 (segment (start 112.1 114.0875) (end 111.6 113.5875) (width 0.1524) (layer "F.Cu") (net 3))
 (segment (start 111.6 113.5875) (end 111.6 112.285) (width 0.1524) (layer "F.Cu") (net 3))
 (segment (start 112.1 112.225) (end 112.1 113.1875) (width 0.1524) (layer "F.Cu") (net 4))
 (segment (start 112.1 113.1875) (end 112.5 113.5875) (width 0.1524) (layer "F.Cu") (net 4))
 (segment (start 113.1 117.6125) (end 113.1 114.1875) (width 0.1524) (layer "F.Cu") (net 4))
 (segment (start 113.1 114.1875) (end 112.5 113.5875) (width 0.1524) (layer "F.Cu") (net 4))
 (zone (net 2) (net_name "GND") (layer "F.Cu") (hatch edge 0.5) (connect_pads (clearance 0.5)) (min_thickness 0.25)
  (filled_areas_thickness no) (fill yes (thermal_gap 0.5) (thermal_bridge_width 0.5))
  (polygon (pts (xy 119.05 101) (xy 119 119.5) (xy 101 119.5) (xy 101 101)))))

